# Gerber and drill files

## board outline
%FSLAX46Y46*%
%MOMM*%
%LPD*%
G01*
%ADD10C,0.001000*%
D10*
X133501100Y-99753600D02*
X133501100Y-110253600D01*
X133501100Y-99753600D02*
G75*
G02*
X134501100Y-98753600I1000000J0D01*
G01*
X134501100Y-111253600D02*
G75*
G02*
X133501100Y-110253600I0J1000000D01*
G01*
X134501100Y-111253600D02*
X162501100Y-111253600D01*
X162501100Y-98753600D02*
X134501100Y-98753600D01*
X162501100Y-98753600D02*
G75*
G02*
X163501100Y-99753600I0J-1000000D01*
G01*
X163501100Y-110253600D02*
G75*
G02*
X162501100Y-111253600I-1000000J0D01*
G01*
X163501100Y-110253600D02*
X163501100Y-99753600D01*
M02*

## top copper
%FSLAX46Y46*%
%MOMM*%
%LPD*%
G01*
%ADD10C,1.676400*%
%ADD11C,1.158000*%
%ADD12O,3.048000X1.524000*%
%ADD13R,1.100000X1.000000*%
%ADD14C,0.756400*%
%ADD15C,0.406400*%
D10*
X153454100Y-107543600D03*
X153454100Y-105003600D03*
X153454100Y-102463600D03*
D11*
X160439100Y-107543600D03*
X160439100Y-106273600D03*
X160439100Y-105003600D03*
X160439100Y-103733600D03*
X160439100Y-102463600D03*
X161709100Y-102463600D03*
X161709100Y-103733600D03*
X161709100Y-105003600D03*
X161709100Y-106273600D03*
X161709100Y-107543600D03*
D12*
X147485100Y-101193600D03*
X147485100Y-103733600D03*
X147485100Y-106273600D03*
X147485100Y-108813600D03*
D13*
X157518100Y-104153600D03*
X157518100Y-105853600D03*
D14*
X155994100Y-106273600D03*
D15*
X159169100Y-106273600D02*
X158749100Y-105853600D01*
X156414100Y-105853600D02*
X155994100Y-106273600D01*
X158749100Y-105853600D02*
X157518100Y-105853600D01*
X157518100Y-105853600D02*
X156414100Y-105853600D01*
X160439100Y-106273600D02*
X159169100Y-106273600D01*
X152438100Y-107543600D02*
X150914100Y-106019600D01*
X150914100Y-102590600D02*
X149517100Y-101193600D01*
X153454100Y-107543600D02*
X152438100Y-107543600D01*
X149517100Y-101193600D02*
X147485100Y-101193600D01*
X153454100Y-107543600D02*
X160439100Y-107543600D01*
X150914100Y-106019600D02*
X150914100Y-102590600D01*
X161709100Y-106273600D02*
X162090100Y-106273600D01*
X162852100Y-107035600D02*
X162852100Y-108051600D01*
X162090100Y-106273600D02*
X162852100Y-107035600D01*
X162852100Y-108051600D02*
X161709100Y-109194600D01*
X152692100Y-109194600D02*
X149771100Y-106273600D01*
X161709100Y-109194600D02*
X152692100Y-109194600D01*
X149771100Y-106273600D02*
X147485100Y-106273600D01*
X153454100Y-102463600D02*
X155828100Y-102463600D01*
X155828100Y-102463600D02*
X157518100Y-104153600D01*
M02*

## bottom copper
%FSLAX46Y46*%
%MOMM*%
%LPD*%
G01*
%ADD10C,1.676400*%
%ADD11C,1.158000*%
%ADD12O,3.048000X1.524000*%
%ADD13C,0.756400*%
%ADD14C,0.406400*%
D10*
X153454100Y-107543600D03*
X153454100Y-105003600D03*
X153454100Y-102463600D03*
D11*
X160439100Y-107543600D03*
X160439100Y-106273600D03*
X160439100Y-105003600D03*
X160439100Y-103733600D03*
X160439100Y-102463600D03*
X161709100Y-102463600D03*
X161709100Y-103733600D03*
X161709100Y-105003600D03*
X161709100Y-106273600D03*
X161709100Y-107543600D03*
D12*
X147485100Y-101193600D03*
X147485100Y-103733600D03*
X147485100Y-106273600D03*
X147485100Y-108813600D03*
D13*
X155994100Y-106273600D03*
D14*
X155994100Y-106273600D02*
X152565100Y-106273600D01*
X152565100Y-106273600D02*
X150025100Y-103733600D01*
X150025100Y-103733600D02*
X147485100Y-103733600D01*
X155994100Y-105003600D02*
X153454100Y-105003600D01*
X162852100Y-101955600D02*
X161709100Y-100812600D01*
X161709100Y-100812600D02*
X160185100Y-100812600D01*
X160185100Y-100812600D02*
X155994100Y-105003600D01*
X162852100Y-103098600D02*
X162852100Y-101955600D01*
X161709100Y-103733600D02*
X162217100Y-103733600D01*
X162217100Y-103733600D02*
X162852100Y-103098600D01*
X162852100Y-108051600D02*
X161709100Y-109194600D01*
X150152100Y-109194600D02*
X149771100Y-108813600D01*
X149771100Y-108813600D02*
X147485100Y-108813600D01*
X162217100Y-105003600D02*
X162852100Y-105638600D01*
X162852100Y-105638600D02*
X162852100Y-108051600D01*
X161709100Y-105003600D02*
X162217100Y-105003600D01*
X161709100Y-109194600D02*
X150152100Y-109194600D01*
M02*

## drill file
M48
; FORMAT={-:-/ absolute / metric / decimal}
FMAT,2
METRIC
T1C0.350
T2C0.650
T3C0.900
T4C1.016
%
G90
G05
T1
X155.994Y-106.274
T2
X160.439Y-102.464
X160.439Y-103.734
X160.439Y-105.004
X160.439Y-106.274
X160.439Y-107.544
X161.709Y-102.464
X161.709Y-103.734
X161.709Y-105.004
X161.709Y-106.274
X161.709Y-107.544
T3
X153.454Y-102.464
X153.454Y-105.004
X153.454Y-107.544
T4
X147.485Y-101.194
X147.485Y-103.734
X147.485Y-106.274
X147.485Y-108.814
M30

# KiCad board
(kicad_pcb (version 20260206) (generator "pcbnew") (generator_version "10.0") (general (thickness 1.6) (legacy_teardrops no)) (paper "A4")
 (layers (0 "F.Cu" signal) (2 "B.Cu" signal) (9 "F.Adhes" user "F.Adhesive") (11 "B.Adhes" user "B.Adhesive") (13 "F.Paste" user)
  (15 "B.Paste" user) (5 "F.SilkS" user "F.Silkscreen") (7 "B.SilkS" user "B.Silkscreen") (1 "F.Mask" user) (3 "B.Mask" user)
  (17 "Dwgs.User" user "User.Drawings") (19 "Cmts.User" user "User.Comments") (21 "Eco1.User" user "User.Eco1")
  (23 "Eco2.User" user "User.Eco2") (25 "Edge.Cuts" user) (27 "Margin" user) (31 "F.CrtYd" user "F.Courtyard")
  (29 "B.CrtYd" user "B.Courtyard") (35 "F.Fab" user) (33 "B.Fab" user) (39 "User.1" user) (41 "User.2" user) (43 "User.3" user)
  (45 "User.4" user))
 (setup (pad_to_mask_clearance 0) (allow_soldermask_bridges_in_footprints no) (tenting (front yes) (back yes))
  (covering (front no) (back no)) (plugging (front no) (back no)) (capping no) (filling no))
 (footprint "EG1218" (layer "F.Cu") (at 153.4541 105.0036 90)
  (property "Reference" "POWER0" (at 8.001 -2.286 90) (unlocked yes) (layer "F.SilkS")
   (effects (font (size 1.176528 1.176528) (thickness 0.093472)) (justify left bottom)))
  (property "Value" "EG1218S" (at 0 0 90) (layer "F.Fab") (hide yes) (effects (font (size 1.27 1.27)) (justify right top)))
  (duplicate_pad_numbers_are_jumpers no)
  (pad "O" thru_hole circle (at -2.54 0 90) (size 1.6764 1.6764) (drill 0.9) (layers "*.Cu" "*.Mask") (remove_unused_layers no) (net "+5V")
   (solder_mask_margin 0.1016) (thermal_bridge_angle 0))
  (pad "P" thru_hole circle (at 0 0 90) (size 1.6764 1.6764) (drill 0.9) (layers "*.Cu" "*.Mask") (remove_unused_layers no) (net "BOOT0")
   (solder_mask_margin 0.1016) (thermal_bridge_angle 0))
  (pad "S" thru_hole circle (at 2.54 0 90) (size 1.6764 1.6764) (drill 0.9) (layers "*.Cu" "*.Mask") (remove_unused_layers no) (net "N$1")
   (solder_mask_margin 0.1016) (thermal_bridge_angle 0)))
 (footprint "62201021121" (layer "F.Cu") (at 161.0741 105.0036 90)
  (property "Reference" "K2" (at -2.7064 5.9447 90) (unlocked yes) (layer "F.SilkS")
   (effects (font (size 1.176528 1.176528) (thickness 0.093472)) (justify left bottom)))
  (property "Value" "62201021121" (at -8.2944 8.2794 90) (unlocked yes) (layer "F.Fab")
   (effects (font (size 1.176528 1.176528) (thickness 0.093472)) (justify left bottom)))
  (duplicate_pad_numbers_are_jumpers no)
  (pad "1" thru_hole circle (at -2.54 -0.635 90) (size 1.158 1.158) (drill 0.65) (layers "*.Cu" "*.Mask") (remove_unused_layers no)
   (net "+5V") (solder_mask_margin 0.1016) (thermal_bridge_angle 0))
  (pad "2" thru_hole circle (at -1.27 -0.635 90) (size 1.158 1.158) (drill 0.65) (layers "*.Cu" "*.Mask") (remove_unused_layers no)
   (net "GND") (solder_mask_margin 0.1016) (thermal_bridge_angle 0))
  (pad "3" thru_hole circle (at 0 -0.635 90) (size 1.158 1.158) (drill 0.65) (layers "*.Cu" "*.Mask") (remove_unused_layers no)
   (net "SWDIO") (solder_mask_margin 0.1016) (thermal_bridge_angle 0))
  (pad "4" thru_hole circle (at 1.27 -0.635 90) (size 1.158 1.158) (drill 0.65) (layers "*.Cu" "*.Mask") (remove_unused_layers no)
   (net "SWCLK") (solder_mask_margin 0.1016) (thermal_bridge_angle 0))
  (pad "5" thru_hole circle (at 2.54 -0.635 90) (size 1.158 1.158) (drill 0.65) (layers "*.Cu" "*.Mask") (remove_unused_layers no)
   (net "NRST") (solder_mask_margin 0.1016) (thermal_bridge_angle 0))
  (pad "6" thru_hole circle (at 2.54 0.635 90) (size 1.158 1.158) (drill 0.65) (layers "*.Cu" "*.Mask") (remove_unused_layers no)
   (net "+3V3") (solder_mask_margin 0.1016) (thermal_bridge_angle 0))
  (pad "7" thru_hole circle (at 1.27 0.635 90) (size 1.158 1.158) (drill 0.65) (layers "*.Cu" "*.Mask") (remove_unused_layers no)
   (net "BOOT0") (solder_mask_margin 0.1016) (thermal_bridge_angle 0))
  (pad "8" thru_hole circle (at 0 0.635 90) (size 1.158 1.158) (drill 0.65) (layers "*.Cu" "*.Mask") (remove_unused_layers no)
   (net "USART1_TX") (solder_mask_margin 0.1016) (thermal_bridge_angle 0))
  (pad "9" thru_hole circle (at -1.27 0.635 90) (size 1.158 1.158) (drill 0.65) (layers "*.Cu" "*.Mask") (remove_unused_layers no)
   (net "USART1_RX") (solder_mask_margin 0.1016) (thermal_bridge_angle 0))
  (pad "10" thru_hole circle (at -2.54 0.635 90) (size 1.158 1.158) (drill 0.65) (layers "*.Cu" "*.Mask") (remove_unused_layers no)
   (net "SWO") (solder_mask_margin 0.1016) (thermal_bridge_angle 0)))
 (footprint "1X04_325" (layer "F.Cu") (at 147.4851 105.0036 -90)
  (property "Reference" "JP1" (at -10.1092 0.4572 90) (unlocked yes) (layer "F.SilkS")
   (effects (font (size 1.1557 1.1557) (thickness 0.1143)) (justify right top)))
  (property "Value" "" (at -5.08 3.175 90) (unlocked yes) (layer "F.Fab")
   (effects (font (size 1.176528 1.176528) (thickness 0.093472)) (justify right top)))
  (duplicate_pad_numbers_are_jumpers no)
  (pad "1" thru_hole oval (at -3.81 0) (size 3.048 1.524) (drill 1.016) (layers "*.Cu" "*.Mask") (remove_unused_layers no) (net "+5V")
   (solder_mask_margin 0.1016) (thermal_bridge_angle 0))
  (pad "2" thru_hole oval (at -1.27 0) (size 3.048 1.524) (drill 1.016) (layers "*.Cu" "*.Mask") (remove_unused_layers no) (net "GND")
   (solder_mask_margin 0.1016) (thermal_bridge_angle 0))
  (pad "3" thru_hole oval (at 1.27 0) (size 3.048 1.524) (drill 1.016) (layers "*.Cu" "*.Mask") (remove_unused_layers no) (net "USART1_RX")
   (solder_mask_margin 0.1016) (thermal_bridge_angle 0))
  (pad "4" thru_hole oval (at 3.81 0) (size 3.048 1.524) (drill 1.016) (layers "*.Cu" "*.Mask") (remove_unused_layers no) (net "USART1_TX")
   (solder_mask_margin 0.1016) (thermal_bridge_angle 0)))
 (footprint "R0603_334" (layer "F.Cu") (at 157.5181 105.0036 -90)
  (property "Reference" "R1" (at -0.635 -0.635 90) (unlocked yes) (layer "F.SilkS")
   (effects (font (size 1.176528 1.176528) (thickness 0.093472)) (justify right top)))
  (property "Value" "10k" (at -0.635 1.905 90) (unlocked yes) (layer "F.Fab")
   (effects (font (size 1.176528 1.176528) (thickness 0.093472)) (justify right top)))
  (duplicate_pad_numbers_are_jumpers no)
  (pad "1" smd rect (at -0.85 0 270) (size 1 1.1) (layers "F.Cu" "F.Mask" "F.Paste") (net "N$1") (solder_mask_margin 0.1016)
   (solder_paste_margin 0) (thermal_bridge_angle 0))
  (pad "2" smd rect (at 0.85 0 270) (size 1 1.1) (layers "F.Cu" "F.Mask" "F.Paste") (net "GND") (solder_mask_margin 0.1016)
   (solder_paste_margin 0) (thermal_bridge_angle 0)))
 (gr_line (start 133.5011 99.7536) (end 133.5011 110.2536) (stroke (width 0.001) (type solid)) (layer "Edge.Cuts"))
 (gr_arc (start 133.5011 99.7536) (mid 133.793993 99.046493) (end 134.5011 98.7536) (stroke (width 0.001) (type solid)) (layer "Edge.Cuts"))
 (gr_arc (start 134.5011 111.2536) (mid 133.793993 110.960707) (end 133.5011 110.2536) (stroke (width 0.001) (type solid))
  (layer "Edge.Cuts"))
 (gr_line (start 134.5011 111.2536) (end 162.5011 111.2536) (stroke (width 0.001) (type solid)) (layer "Edge.Cuts"))
 (gr_line (start 162.5011 98.7536) (end 134.5011 98.7536) (stroke (width 0.001) (type solid)) (layer "Edge.Cuts"))
 (gr_arc (start 162.5011 98.7536) (mid 163.208207 99.046493) (end 163.5011 99.7536) (stroke (width 0.001) (type solid)) (layer "Edge.Cuts"))
 (gr_arc (start 163.5011 110.2536) (mid 163.208207 110.960707) (end 162.5011 111.2536) (stroke (width 0.001) (type solid))
  (layer "Edge.Cuts"))
 (gr_line (start 163.5011 110.2536) (end 163.5011 99.7536) (stroke (width 0.001) (type solid)) (layer "Edge.Cuts"))
 (segment (start 159.1691 106.2736) (end 158.7491 105.8536) (width 0.4064) (layer "F.Cu") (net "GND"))
 (segment (start 156.4141 105.8536) (end 155.9941 106.2736) (width 0.4064) (layer "F.Cu") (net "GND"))
 (segment (start 158.7491 105.8536) (end 157.5181 105.8536) (width 0.4064) (layer "F.Cu") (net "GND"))
 (segment (start 157.5181 105.8536) (end 156.4141 105.8536) (width 0.4064) (layer "F.Cu") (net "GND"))
 (segment (start 160.4391 106.2736) (end 159.1691 106.2736) (width 0.4064) (layer "F.Cu") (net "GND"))
 (via (at 155.9941 106.2736) (size 0.7564) (drill 0.35) (layers "F.Cu" "B.Cu") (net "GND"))
 (segment (start 155.9941 106.2736) (end 152.5651 106.2736) (width 0.4064) (layer "B.Cu") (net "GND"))
 (segment (start 152.5651 106.2736) (end 150.0251 103.7336) (width 0.4064) (layer "B.Cu") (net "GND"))
 (segment (start 150.0251 103.7336) (end 147.4851 103.7336) (width 0.4064) (layer "B.Cu") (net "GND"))
 (segment (start 152.4381 107.5436) (end 150.9141 106.0196) (width 0.4064) (layer "F.Cu") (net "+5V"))
 (segment (start 150.9141 102.5906) (end 149.5171 101.1936) (width 0.4064) (layer "F.Cu") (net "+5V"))
 (segment (start 153.4541 107.5436) (end 152.4381 107.5436) (width 0.4064) (layer "F.Cu") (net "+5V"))
 (segment (start 149.5171 101.1936) (end 147.4851 101.1936) (width 0.4064) (layer "F.Cu") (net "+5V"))
 (segment (start 153.4541 107.5436) (end 160.4391 107.5436) (width 0.4064) (layer "F.Cu") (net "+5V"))
 (segment (start 150.9141 106.0196) (end 150.9141 102.5906) (width 0.4064) (layer "F.Cu") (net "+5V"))
 (segment (start 155.9941 105.0036) (end 153.4541 105.0036) (width 0.4064) (layer "B.Cu") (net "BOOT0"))
 (segment (start 162.8521 101.9556) (end 161.7091 100.8126) (width 0.4064) (layer "B.Cu") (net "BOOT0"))
 (segment (start 161.7091 100.8126) (end 160.1851 100.8126) (width 0.4064) (layer "B.Cu") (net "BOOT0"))
 (segment (start 160.1851 100.8126) (end 155.9941 105.0036) (width 0.4064) (layer "B.Cu") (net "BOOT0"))
 (segment (start 162.8521 103.0986) (end 162.8521 101.9556) (width 0.4064) (layer "B.Cu") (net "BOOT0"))
 (segment (start 161.7091 103.7336) (end 162.2171 103.7336) (width 0.4064) (layer "B.Cu") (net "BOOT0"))
 (segment (start 162.2171 103.7336) (end 162.8521 103.0986) (width 0.4064) (layer "B.Cu") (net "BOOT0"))
 (segment (start 162.8521 108.0516) (end 161.7091 109.1946) (width 0.4064) (layer "B.Cu") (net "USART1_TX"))
 (segment (start 150.1521 109.1946) (end 149.7711 108.8136) (width 0.4064) (layer "B.Cu") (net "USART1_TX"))
 (segment (start 149.7711 108.8136) (end 147.4851 108.8136) (width 0.4064) (layer "B.Cu") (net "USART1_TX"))
 (segment (start 162.2171 105.0036) (end 162.8521 105.6386) (width 0.4064) (layer "B.Cu") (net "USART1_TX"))
 (segment (start 162.8521 105.6386) (end 162.8521 108.0516) (width 0.4064) (layer "B.Cu") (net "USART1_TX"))
 (segment (start 161.7091 105.0036) (end 162.2171 105.0036) (width 0.4064) (layer "B.Cu") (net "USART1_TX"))
 (segment (start 161.7091 109.1946) (end 150.1521 109.1946) (width 0.4064) (layer "B.Cu") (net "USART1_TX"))
 (segment (start 161.7091 106.2736) (end 162.0901 106.2736) (width 0.4064) (layer "F.Cu") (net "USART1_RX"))
 (segment (start 162.8521 107.0356) (end 162.8521 108.0516) (width 0.4064) (layer "F.Cu") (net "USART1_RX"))
 (segment (start 162.0901 106.2736) (end 162.8521 107.0356) (width 0.4064) (layer "F.Cu") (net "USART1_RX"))
 (segment (start 162.8521 108.0516) (end 161.7091 109.1946) (width 0.4064) (layer "F.Cu") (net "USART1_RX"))
 (segment (start 152.6921 109.1946) (end 149.7711 106.2736) (width 0.4064) (layer "F.Cu") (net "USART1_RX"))
 (segment (start 161.7091 109.1946) (end 152.6921 109.1946) (width 0.4064) (layer "F.Cu") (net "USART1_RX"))
 (segment (start 149.7711 106.2736) (end 147.4851 106.2736) (width 0.4064) (layer "F.Cu") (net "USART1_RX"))
 (segment (start 153.4541 102.4636) (end 155.8281 102.4636) (width 0.4064) (layer "F.Cu") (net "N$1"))
 (segment (start 155.8281 102.4636) (end 157.5181 104.1536) (width 0.4064) (layer "F.Cu") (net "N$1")))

